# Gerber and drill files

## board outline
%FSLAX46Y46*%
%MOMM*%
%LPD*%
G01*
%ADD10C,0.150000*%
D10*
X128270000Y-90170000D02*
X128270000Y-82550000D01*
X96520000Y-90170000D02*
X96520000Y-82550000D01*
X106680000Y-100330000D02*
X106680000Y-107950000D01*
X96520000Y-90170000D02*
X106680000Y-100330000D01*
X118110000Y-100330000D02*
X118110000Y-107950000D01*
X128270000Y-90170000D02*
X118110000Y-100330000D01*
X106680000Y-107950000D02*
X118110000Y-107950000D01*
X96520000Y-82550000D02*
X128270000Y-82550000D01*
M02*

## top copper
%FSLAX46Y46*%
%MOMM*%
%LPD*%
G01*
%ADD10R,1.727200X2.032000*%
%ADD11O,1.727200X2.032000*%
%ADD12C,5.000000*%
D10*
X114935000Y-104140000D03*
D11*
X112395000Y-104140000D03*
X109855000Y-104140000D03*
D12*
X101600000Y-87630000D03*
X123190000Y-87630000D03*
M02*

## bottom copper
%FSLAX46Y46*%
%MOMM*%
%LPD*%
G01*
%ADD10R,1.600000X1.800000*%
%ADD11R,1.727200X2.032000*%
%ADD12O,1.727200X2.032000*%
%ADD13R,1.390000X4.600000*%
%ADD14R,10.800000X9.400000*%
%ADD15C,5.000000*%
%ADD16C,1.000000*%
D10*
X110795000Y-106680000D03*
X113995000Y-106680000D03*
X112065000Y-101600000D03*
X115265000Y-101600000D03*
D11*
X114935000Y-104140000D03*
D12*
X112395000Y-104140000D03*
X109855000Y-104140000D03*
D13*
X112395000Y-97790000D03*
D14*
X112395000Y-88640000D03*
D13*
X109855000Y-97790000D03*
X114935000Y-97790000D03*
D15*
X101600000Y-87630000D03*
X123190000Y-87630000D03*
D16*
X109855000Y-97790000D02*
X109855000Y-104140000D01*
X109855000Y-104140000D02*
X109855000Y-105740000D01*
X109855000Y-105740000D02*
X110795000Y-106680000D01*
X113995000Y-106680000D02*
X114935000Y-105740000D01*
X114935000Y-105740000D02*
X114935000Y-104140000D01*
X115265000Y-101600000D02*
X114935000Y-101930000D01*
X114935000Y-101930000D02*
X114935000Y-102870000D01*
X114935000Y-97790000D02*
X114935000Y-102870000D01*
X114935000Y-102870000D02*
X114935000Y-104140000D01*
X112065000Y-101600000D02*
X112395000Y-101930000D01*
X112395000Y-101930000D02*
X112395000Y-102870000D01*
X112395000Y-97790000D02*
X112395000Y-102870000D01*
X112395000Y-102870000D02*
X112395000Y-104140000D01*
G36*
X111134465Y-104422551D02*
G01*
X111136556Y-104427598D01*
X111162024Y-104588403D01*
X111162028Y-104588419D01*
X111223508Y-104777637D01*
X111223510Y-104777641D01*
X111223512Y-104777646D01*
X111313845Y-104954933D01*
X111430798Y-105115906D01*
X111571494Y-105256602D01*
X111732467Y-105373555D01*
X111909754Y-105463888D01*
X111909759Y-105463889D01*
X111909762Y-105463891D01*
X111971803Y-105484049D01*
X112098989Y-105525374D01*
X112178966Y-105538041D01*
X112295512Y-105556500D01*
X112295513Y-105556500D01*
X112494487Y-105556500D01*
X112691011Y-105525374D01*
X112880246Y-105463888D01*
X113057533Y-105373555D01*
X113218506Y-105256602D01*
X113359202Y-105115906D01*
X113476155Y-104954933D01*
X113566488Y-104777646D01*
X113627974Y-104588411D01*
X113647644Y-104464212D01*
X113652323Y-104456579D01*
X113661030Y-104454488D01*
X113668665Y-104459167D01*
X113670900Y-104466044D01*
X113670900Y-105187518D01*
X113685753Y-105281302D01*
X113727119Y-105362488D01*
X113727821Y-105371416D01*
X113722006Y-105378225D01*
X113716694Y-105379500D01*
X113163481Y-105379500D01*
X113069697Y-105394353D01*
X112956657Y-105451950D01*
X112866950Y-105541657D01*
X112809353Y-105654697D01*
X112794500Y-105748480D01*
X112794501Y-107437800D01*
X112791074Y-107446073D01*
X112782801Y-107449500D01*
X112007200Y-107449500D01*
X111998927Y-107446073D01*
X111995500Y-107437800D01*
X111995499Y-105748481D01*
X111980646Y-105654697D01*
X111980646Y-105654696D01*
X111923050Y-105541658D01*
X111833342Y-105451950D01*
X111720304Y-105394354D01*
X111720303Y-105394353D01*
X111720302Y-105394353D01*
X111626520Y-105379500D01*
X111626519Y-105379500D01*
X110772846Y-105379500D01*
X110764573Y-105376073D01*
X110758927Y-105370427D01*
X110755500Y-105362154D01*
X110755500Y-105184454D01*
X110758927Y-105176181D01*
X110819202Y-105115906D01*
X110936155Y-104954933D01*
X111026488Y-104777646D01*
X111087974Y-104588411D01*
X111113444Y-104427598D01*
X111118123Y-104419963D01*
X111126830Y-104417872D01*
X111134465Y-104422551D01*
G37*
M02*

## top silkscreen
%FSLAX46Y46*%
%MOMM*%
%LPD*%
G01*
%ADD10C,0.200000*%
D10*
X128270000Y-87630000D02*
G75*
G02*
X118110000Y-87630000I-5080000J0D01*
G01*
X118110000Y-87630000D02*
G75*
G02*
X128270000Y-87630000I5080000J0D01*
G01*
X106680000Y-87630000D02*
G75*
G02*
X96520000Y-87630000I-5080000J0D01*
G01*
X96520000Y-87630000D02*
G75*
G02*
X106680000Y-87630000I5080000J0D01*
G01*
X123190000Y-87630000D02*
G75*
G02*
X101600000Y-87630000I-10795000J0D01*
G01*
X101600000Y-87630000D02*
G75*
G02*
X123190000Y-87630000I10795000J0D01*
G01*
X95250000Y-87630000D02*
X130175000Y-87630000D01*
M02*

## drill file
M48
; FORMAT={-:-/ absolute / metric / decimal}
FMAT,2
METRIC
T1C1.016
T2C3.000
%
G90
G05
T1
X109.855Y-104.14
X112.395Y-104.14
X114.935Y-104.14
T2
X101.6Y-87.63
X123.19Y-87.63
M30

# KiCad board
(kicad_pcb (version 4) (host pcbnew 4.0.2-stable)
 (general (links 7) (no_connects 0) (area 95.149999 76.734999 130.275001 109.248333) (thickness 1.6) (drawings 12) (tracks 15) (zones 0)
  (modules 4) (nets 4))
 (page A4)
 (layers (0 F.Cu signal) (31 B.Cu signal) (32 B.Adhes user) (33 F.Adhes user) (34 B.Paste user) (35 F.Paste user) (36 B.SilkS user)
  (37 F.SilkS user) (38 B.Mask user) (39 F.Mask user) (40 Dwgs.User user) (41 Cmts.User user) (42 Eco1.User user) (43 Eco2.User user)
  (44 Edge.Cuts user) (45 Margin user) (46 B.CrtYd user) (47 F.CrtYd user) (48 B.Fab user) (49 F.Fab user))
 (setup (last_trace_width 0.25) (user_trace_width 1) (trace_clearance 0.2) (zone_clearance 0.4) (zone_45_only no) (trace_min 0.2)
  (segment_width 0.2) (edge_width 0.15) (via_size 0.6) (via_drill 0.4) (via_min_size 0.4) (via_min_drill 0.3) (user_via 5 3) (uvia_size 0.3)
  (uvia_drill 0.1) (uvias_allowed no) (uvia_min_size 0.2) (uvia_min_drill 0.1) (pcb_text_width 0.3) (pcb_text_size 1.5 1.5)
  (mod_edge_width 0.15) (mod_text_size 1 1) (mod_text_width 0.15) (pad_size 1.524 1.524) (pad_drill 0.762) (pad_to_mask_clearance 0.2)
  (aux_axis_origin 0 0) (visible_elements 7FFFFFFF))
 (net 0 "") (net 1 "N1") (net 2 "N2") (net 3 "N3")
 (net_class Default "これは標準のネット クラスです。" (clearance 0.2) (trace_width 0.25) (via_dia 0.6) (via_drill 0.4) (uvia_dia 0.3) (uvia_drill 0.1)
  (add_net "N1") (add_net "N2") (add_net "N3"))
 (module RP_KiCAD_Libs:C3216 (layer B.Cu) (at 112.395 106.68)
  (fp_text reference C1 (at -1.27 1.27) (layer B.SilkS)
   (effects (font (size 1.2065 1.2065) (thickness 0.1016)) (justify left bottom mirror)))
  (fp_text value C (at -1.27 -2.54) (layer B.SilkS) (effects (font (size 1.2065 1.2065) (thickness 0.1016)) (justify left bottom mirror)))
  (pad 1 smd rect (at -1.6 0) (size 1.6 1.8) (layers B.Cu B.Paste B.Mask) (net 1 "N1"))
  (pad 2 smd rect (at 1.6 0) (size 1.6 1.8) (layers B.Cu B.Paste B.Mask) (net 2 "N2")))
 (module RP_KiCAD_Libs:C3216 (layer B.Cu) (at 113.665 101.6)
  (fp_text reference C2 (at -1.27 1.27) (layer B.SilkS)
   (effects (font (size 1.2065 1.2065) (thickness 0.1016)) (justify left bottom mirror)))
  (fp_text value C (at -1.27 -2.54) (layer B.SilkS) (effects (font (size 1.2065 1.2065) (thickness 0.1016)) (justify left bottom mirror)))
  (pad 1 smd rect (at -1.6 0) (size 1.6 1.8) (layers B.Cu B.Paste B.Mask) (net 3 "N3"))
  (pad 2 smd rect (at 1.6 0) (size 1.6 1.8) (layers B.Cu B.Paste B.Mask) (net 2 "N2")))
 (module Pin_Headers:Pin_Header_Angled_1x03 (layer B.Cu) (at 114.935 104.14 90)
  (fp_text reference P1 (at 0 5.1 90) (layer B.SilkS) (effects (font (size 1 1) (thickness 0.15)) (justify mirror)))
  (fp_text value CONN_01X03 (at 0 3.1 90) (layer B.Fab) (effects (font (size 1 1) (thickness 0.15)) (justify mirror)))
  (pad 1 thru_hole rect (at 0 0 90) (size 2.032 1.7272) (drill 1.016) (layers *.Cu *.Mask B.SilkS) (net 2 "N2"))
  (pad 2 thru_hole oval (at 0 -2.54 90) (size 2.032 1.7272) (drill 1.016) (layers *.Cu *.Mask B.SilkS) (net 3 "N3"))
  (pad 3 thru_hole oval (at 0 -5.08 90) (size 2.032 1.7272) (drill 1.016) (layers *.Cu *.Mask B.SilkS) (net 1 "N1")))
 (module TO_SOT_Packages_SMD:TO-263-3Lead (layer B.Cu) (at 112.395 97.79 90)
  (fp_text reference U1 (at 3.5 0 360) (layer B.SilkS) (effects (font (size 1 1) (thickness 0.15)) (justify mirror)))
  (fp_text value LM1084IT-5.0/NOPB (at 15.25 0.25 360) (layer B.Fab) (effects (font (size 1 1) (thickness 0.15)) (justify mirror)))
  (pad 2 smd rect (at 0 0 90) (size 4.6 1.39) (layers B.Cu B.Paste B.Mask) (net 3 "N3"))
  (pad 4 smd rect (at 9.15 0 90) (size 9.4 10.8) (layers B.Cu B.Paste B.Mask))
  (pad 3 smd rect (at 0 -2.54 90) (size 4.6 1.39) (layers B.Cu B.Paste B.Mask) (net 1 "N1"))
  (pad 1 smd rect (at 0 2.54 90) (size 4.6 1.39) (layers B.Cu B.Paste B.Mask) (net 2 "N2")))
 (gr_line (start 128.27 90.17) (end 128.27 82.55) (angle 90) (layer Edge.Cuts) (width 0.15))
 (gr_line (start 96.52 90.17) (end 96.52 82.55) (angle 90) (layer Edge.Cuts) (width 0.15))
 (gr_line (start 106.68 100.33) (end 106.68 107.95) (angle 90) (layer Edge.Cuts) (width 0.15))
 (gr_line (start 96.52 90.17) (end 106.68 100.33) (angle 90) (layer Edge.Cuts) (width 0.15))
 (gr_line (start 118.11 100.33) (end 118.11 107.95) (angle 90) (layer Edge.Cuts) (width 0.15))
 (gr_line (start 128.27 90.17) (end 118.11 100.33) (angle 90) (layer Edge.Cuts) (width 0.15))
 (gr_line (start 106.68 107.95) (end 118.11 107.95) (angle 90) (layer Edge.Cuts) (width 0.15))
 (gr_line (start 96.52 82.55) (end 128.27 82.55) (angle 90) (layer Edge.Cuts) (width 0.15))
 (gr_circle (center 123.19 87.63) (end 118.11 87.63) (layer F.SilkS) (width 0.2))
 (gr_circle (center 101.6 87.63) (end 106.68 87.63) (layer F.SilkS) (width 0.2))
 (gr_circle (center 112.395 87.63) (end 123.19 87.63) (layer F.SilkS) (width 0.2))
 (gr_line (start 95.25 87.63) (end 130.175 87.63) (angle 90) (layer F.SilkS) (width 0.2))
 (via (at 101.6 87.63) (size 5) (drill 3) (layers F.Cu B.Cu) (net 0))
 (via (at 123.19 87.63) (size 5) (drill 3) (layers F.Cu B.Cu) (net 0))
 (segment (start 109.855 97.79) (end 109.855 104.14) (width 1) (layer B.Cu) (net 1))
 (segment (start 109.855 104.14) (end 109.855 105.74) (width 1) (layer B.Cu) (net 1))
 (segment (start 109.855 105.74) (end 110.795 106.68) (width 1) (layer B.Cu) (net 1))
 (segment (start 113.995 106.68) (end 114.935 105.74) (width 1) (layer B.Cu) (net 2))
 (segment (start 114.935 105.74) (end 114.935 104.14) (width 1) (layer B.Cu) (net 2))
 (segment (start 115.265 101.6) (end 114.935 101.93) (width 1) (layer B.Cu) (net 2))
 (segment (start 114.935 101.93) (end 114.935 102.87) (width 1) (layer B.Cu) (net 2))
 (segment (start 114.935 97.79) (end 114.935 102.87) (width 1) (layer B.Cu) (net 2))
 (segment (start 114.935 102.87) (end 114.935 104.14) (width 1) (layer B.Cu) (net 2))
 (segment (start 112.065 101.6) (end 112.395 101.93) (width 1) (layer B.Cu) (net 3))
 (segment (start 112.395 101.93) (end 112.395 102.87) (width 1) (layer B.Cu) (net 3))
 (segment (start 112.395 97.79) (end 112.395 102.87) (width 1) (layer B.Cu) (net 3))
 (segment (start 112.395 102.87) (end 112.395 104.14) (width 1) (layer B.Cu) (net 3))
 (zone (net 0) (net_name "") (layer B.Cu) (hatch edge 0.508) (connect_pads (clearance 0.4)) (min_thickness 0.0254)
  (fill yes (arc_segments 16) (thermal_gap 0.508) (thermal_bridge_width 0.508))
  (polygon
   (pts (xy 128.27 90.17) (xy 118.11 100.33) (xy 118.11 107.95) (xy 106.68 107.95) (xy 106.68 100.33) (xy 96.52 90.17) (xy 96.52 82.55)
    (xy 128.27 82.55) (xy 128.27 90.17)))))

